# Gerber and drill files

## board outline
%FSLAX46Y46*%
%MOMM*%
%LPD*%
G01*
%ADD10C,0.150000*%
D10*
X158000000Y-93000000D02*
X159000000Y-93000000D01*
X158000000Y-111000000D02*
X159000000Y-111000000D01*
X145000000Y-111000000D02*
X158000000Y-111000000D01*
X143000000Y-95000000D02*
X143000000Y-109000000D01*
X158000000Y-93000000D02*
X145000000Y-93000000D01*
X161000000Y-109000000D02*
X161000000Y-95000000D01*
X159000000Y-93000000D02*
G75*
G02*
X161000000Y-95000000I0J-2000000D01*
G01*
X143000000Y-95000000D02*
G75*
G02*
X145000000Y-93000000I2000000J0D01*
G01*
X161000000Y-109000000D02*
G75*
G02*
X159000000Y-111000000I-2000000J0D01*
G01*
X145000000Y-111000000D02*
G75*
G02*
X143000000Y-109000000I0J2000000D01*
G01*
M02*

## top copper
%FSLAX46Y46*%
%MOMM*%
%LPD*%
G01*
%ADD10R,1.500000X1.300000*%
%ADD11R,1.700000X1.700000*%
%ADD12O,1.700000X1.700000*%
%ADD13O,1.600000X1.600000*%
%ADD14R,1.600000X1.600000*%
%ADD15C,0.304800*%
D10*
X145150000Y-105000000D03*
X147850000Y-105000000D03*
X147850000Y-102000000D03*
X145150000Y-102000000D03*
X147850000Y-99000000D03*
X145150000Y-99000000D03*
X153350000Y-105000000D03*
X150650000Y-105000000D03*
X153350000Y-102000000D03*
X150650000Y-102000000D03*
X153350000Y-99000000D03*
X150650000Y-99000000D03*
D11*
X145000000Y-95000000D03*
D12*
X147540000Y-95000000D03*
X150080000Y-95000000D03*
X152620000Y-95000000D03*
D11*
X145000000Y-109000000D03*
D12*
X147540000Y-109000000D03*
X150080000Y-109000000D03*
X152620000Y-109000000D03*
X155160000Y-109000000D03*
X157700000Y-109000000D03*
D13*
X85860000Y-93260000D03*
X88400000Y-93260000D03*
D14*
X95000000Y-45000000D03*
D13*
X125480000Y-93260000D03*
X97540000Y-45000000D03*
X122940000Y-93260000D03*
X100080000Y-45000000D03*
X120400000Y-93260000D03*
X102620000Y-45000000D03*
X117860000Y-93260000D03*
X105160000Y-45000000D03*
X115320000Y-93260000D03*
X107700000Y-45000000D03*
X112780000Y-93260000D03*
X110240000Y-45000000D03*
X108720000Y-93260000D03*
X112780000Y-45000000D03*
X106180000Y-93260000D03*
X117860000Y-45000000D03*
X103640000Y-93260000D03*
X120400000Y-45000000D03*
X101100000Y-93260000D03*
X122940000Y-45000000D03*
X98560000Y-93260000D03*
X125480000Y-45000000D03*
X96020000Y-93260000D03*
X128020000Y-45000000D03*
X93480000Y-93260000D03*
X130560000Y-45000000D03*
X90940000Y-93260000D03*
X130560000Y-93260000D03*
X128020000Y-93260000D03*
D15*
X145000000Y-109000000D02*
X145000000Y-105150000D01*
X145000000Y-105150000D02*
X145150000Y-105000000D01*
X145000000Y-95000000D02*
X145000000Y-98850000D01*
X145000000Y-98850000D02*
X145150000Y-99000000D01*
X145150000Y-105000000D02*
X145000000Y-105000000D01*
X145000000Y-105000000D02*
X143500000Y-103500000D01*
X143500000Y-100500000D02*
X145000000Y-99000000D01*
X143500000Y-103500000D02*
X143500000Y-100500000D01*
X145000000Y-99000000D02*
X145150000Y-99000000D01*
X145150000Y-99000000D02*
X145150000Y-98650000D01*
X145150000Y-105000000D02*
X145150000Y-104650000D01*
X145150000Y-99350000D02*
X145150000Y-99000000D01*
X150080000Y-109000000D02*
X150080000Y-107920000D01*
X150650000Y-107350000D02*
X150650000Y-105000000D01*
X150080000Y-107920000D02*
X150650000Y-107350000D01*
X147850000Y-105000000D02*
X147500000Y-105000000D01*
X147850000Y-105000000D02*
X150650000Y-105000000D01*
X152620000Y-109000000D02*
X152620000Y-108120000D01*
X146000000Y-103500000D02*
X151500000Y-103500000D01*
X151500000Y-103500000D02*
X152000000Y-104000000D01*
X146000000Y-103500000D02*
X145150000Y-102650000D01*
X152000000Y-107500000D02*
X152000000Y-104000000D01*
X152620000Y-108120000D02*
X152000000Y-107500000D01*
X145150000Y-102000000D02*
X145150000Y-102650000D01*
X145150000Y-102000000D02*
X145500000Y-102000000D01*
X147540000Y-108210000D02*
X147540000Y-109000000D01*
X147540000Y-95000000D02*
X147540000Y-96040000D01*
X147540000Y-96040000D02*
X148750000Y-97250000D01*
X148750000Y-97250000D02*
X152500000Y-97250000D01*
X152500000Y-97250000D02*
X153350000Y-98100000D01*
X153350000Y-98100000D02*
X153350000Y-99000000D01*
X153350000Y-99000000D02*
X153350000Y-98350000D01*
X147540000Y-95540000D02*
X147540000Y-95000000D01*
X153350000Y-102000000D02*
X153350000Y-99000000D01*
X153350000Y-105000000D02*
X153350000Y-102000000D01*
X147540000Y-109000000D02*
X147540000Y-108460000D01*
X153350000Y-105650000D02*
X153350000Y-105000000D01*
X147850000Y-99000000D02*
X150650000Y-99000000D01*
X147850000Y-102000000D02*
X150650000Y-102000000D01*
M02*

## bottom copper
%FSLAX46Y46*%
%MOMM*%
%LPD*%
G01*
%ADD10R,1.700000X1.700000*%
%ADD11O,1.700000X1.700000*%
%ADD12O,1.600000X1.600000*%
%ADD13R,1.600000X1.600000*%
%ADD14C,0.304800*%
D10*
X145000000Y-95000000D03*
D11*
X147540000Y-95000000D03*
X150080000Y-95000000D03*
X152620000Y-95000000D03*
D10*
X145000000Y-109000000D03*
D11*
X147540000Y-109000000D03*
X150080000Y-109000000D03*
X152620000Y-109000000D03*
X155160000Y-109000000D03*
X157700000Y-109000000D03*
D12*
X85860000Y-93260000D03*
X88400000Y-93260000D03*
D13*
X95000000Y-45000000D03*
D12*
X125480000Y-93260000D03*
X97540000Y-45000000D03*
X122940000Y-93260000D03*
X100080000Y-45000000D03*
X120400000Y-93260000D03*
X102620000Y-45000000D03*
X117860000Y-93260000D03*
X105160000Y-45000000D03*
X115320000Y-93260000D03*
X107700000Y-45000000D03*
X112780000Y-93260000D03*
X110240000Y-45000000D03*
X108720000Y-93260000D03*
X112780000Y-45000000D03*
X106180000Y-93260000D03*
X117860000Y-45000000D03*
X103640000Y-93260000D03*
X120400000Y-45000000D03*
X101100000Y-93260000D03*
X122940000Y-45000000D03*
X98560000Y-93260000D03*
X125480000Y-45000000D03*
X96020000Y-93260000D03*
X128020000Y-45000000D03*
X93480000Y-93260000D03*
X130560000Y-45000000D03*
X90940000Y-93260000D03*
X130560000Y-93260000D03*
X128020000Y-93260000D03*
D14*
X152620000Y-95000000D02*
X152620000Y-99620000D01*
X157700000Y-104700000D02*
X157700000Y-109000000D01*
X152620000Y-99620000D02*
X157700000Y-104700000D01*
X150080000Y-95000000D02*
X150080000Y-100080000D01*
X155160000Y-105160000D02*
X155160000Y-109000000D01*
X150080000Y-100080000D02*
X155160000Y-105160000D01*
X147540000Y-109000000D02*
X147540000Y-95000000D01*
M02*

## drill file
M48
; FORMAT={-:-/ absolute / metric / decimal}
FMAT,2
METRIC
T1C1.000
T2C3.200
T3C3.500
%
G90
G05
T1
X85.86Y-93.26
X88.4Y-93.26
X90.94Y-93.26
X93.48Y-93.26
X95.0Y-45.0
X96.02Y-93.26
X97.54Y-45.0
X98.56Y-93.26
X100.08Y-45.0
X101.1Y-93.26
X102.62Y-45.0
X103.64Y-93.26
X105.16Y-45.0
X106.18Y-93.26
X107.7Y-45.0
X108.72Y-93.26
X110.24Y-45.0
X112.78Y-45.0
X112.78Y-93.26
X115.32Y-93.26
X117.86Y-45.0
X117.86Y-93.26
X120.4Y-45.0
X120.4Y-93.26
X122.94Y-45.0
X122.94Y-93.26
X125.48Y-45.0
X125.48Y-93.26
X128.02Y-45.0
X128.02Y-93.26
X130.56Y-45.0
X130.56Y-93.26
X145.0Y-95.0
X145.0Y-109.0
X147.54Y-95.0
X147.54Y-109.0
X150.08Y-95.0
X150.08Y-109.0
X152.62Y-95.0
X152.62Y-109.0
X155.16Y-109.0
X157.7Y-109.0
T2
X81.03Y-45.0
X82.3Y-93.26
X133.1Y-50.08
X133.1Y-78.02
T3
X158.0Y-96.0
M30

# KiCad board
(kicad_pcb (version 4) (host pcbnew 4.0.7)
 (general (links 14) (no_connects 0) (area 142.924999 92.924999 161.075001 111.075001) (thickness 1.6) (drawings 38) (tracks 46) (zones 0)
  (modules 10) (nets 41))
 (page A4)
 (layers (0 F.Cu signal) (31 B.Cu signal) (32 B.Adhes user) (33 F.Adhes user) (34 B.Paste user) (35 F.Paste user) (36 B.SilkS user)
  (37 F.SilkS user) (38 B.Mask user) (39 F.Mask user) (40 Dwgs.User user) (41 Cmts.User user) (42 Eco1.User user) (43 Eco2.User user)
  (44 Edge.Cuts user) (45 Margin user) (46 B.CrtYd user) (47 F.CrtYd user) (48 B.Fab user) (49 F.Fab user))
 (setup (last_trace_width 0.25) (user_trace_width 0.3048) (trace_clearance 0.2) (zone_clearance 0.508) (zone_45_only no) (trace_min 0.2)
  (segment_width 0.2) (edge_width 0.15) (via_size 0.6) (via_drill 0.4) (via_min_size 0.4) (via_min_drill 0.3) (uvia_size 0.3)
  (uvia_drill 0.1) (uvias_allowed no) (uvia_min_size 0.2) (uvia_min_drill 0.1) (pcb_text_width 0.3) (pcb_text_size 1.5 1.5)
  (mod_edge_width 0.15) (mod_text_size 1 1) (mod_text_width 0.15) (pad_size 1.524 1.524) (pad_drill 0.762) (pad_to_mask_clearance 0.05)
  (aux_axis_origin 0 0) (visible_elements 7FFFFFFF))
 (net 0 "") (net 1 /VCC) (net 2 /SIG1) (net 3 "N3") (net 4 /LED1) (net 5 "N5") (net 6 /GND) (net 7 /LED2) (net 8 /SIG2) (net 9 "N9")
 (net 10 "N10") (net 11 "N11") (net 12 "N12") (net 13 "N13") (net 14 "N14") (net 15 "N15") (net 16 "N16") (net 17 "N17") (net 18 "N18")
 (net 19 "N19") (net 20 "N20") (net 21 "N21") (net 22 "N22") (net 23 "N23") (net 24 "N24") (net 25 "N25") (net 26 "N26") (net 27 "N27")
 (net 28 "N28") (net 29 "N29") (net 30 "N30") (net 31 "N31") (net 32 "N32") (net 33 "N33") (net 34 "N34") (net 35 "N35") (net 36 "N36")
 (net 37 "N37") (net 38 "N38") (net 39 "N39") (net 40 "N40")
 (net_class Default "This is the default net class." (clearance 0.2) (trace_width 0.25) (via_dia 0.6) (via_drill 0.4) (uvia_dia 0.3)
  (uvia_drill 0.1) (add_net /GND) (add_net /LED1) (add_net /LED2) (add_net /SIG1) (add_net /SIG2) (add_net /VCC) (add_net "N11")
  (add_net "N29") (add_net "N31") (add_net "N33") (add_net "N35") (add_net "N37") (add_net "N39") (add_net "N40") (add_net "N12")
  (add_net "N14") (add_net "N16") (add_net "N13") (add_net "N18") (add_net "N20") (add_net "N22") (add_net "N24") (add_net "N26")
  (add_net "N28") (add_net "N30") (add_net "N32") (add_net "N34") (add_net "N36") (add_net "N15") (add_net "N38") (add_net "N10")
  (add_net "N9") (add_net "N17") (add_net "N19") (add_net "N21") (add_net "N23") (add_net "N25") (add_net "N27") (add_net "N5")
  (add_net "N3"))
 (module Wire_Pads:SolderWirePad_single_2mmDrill (layer F.Cu) (at 158 96)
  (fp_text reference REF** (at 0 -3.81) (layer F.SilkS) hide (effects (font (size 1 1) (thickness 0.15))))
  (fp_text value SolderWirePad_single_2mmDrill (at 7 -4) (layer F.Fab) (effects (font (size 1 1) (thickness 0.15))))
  (pad "" np_thru_hole circle (at 0 0) (size 3.5 3.5) (drill 3.5) (layers *.Cu *.Mask)))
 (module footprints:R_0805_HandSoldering (layer F.Cu) (at 146.5 105)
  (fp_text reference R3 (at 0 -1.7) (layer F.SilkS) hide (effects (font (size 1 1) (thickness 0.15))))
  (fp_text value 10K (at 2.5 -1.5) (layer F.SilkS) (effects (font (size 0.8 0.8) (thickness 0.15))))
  (pad 1 smd rect (at -1.35 0) (size 1.5 1.3) (layers F.Cu F.Paste F.Mask) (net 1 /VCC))
  (pad 2 smd rect (at 1.35 0) (size 1.5 1.3) (layers F.Cu F.Paste F.Mask) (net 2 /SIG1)))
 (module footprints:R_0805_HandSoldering (layer F.Cu) (at 146.5 102 180)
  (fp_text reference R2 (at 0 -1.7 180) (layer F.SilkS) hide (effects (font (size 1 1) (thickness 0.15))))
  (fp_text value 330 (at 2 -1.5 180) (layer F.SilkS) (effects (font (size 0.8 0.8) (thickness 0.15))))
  (pad 1 smd rect (at -1.35 0 180) (size 1.5 1.3) (layers F.Cu F.Paste F.Mask) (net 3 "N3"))
  (pad 2 smd rect (at 1.35 0 180) (size 1.5 1.3) (layers F.Cu F.Paste F.Mask) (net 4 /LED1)))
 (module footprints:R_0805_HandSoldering (layer F.Cu) (at 146.5 99 180)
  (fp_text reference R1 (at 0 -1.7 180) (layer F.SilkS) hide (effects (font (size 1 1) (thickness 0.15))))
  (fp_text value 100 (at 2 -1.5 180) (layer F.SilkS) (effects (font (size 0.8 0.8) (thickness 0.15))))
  (pad 1 smd rect (at -1.35 0 180) (size 1.5 1.3) (layers F.Cu F.Paste F.Mask) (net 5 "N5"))
  (pad 2 smd rect (at 1.35 0 180) (size 1.5 1.3) (layers F.Cu F.Paste F.Mask) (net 1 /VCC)))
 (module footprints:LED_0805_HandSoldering (layer F.Cu) (at 152 105 180)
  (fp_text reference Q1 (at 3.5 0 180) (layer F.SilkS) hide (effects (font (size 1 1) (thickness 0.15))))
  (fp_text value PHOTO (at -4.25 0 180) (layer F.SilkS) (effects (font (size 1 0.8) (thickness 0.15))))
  (pad 1 smd rect (at -1.35 0 180) (size 1.5 1.3) (layers F.Cu F.Paste F.Mask) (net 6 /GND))
  (pad 2 smd rect (at 1.35 0 180) (size 1.5 1.3) (layers F.Cu F.Paste F.Mask) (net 2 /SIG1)))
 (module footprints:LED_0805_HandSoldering (layer F.Cu) (at 152 102 180)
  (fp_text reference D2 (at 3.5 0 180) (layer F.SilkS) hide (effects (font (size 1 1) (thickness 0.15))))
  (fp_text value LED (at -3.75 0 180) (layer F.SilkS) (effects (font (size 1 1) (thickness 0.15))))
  (pad 1 smd rect (at -1.35 0 180) (size 1.5 1.3) (layers F.Cu F.Paste F.Mask) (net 6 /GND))
  (pad 2 smd rect (at 1.35 0 180) (size 1.5 1.3) (layers F.Cu F.Paste F.Mask) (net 3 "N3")))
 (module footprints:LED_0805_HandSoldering (layer F.Cu) (at 152 99 180)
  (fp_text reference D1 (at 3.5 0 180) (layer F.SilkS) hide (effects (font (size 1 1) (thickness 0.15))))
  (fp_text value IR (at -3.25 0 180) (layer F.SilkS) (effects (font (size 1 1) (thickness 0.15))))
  (pad 1 smd rect (at -1.35 0 180) (size 1.5 1.3) (layers F.Cu F.Paste F.Mask) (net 6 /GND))
  (pad 2 smd rect (at 1.35 0 180) (size 1.5 1.3) (layers F.Cu F.Paste F.Mask) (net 5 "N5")))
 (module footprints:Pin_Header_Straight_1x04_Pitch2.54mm (layer F.Cu) (at 145 95 90)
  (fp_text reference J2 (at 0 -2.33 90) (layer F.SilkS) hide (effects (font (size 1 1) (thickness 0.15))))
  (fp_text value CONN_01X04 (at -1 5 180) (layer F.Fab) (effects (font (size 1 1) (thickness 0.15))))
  (pad 1 thru_hole rect (at 0 0 90) (size 1.7 1.7) (drill 1) (layers *.Cu *.Mask) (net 1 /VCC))
  (pad 2 thru_hole oval (at 0 2.54 90) (size 1.7 1.7) (drill 1) (layers *.Cu *.Mask) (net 6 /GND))
  (pad 3 thru_hole oval (at 0 5.08 90) (size 1.7 1.7) (drill 1) (layers *.Cu *.Mask) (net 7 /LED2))
  (pad 4 thru_hole oval (at 0 7.62 90) (size 1.7 1.7) (drill 1) (layers *.Cu *.Mask) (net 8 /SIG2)))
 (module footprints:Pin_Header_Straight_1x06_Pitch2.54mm (layer F.Cu) (at 145 109 90)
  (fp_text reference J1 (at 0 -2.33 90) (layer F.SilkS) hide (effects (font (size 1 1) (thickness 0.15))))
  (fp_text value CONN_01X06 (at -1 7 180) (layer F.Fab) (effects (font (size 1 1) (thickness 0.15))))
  (pad 1 thru_hole rect (at 0 0 90) (size 1.7 1.7) (drill 1) (layers *.Cu *.Mask) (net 1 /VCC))
  (pad 2 thru_hole oval (at 0 2.54 90) (size 1.7 1.7) (drill 1) (layers *.Cu *.Mask) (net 6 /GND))
  (pad 3 thru_hole oval (at 0 5.08 90) (size 1.7 1.7) (drill 1) (layers *.Cu *.Mask) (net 2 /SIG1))
  (pad 4 thru_hole oval (at 0 7.62 90) (size 1.7 1.7) (drill 1) (layers *.Cu *.Mask) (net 4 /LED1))
  (pad 5 thru_hole oval (at 0 10.16 90) (size 1.7 1.7) (drill 1) (layers *.Cu *.Mask) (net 7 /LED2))
  (pad 6 thru_hole oval (at 0 12.7 90) (size 1.7 1.7) (drill 1) (layers *.Cu *.Mask) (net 8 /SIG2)))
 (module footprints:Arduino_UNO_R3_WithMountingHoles (layer F.Cu) (at 95 45)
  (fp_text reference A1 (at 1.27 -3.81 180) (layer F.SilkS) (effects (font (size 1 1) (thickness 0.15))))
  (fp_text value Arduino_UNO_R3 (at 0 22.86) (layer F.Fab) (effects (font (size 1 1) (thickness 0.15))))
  (pad 32 thru_hole oval (at -9.14 48.26 90) (size 1.6 1.6) (drill 1) (layers *.Cu *.Mask) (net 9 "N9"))
  (pad 31 thru_hole oval (at -6.6 48.26 90) (size 1.6 1.6) (drill 1) (layers *.Cu *.Mask) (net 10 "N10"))
  (pad 1 thru_hole rect (at 0 0 90) (size 1.6 1.6) (drill 1) (layers *.Cu *.Mask) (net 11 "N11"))
  (pad 17 thru_hole oval (at 30.48 48.26 90) (size 1.6 1.6) (drill 1) (layers *.Cu *.Mask) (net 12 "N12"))
  (pad 2 thru_hole oval (at 2.54 0 90) (size 1.6 1.6) (drill 1) (layers *.Cu *.Mask) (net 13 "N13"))
  (pad 18 thru_hole oval (at 27.94 48.26 90) (size 1.6 1.6) (drill 1) (layers *.Cu *.Mask) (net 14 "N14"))
  (pad 3 thru_hole oval (at 5.08 0 90) (size 1.6 1.6) (drill 1) (layers *.Cu *.Mask) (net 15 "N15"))
  (pad 19 thru_hole oval (at 25.4 48.26 90) (size 1.6 1.6) (drill 1) (layers *.Cu *.Mask) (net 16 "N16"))
  (pad 4 thru_hole oval (at 7.62 0 90) (size 1.6 1.6) (drill 1) (layers *.Cu *.Mask) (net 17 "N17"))
  (pad 20 thru_hole oval (at 22.86 48.26 90) (size 1.6 1.6) (drill 1) (layers *.Cu *.Mask) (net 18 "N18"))
  (pad 5 thru_hole oval (at 10.16 0 90) (size 1.6 1.6) (drill 1) (layers *.Cu *.Mask) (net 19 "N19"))
  (pad 21 thru_hole oval (at 20.32 48.26 90) (size 1.6 1.6) (drill 1) (layers *.Cu *.Mask) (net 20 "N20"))
  (pad 6 thru_hole oval (at 12.7 0 90) (size 1.6 1.6) (drill 1) (layers *.Cu *.Mask) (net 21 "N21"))
  (pad 22 thru_hole oval (at 17.78 48.26 90) (size 1.6 1.6) (drill 1) (layers *.Cu *.Mask) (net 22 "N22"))
  (pad 7 thru_hole oval (at 15.24 0 90) (size 1.6 1.6) (drill 1) (layers *.Cu *.Mask) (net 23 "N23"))
  (pad 23 thru_hole oval (at 13.72 48.26 90) (size 1.6 1.6) (drill 1) (layers *.Cu *.Mask) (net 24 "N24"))
  (pad 8 thru_hole oval (at 17.78 0 90) (size 1.6 1.6) (drill 1) (layers *.Cu *.Mask) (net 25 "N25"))
  (pad 24 thru_hole oval (at 11.18 48.26 90) (size 1.6 1.6) (drill 1) (layers *.Cu *.Mask) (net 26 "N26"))
  (pad 9 thru_hole oval (at 22.86 0 90) (size 1.6 1.6) (drill 1) (layers *.Cu *.Mask) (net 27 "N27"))
  (pad 25 thru_hole oval (at 8.64 48.26 90) (size 1.6 1.6) (drill 1) (layers *.Cu *.Mask) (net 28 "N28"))
  (pad 10 thru_hole oval (at 25.4 0 90) (size 1.6 1.6) (drill 1) (layers *.Cu *.Mask) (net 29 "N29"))
  (pad 26 thru_hole oval (at 6.1 48.26 90) (size 1.6 1.6) (drill 1) (layers *.Cu *.Mask) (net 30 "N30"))
  (pad 11 thru_hole oval (at 27.94 0 90) (size 1.6 1.6) (drill 1) (layers *.Cu *.Mask) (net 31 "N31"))
  (pad 27 thru_hole oval (at 3.56 48.26 90) (size 1.6 1.6) (drill 1) (layers *.Cu *.Mask) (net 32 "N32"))
  (pad 12 thru_hole oval (at 30.48 0 90) (size 1.6 1.6) (drill 1) (layers *.Cu *.Mask) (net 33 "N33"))
  (pad 28 thru_hole oval (at 1.02 48.26 90) (size 1.6 1.6) (drill 1) (layers *.Cu *.Mask) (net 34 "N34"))
  (pad 13 thru_hole oval (at 33.02 0 90) (size 1.6 1.6) (drill 1) (layers *.Cu *.Mask) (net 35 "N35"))
  (pad 29 thru_hole oval (at -1.52 48.26 90) (size 1.6 1.6) (drill 1) (layers *.Cu *.Mask) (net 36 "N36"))
  (pad 14 thru_hole oval (at 35.56 0 90) (size 1.6 1.6) (drill 1) (layers *.Cu *.Mask) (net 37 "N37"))
  (pad 30 thru_hole oval (at -4.06 48.26 90) (size 1.6 1.6) (drill 1) (layers *.Cu *.Mask) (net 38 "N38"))
  (pad 15 thru_hole oval (at 35.56 48.26 90) (size 1.6 1.6) (drill 1) (layers *.Cu *.Mask) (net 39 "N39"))
  (pad 16 thru_hole oval (at 33.02 48.26 90) (size 1.6 1.6) (drill 1) (layers *.Cu *.Mask) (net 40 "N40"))
  (pad "" np_thru_hole circle (at -13.97 0 90) (size 3.2 3.2) (drill 3.2) (layers *.Cu *.Mask))
  (pad "" np_thru_hole circle (at -12.7 48.26 90) (size 3.2 3.2) (drill 3.2) (layers *.Cu *.Mask))
  (pad "" np_thru_hole circle (at 38.1 33.02 90) (size 3.2 3.2) (drill 3.2) (layers *.Cu *.Mask))
  (pad "" np_thru_hole circle (at 38.1 5.08 90) (size 3.2 3.2) (drill 3.2) (layers *.Cu *.Mask)))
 (gr_line (start 158 93) (end 159 93) (angle 90) (layer Edge.Cuts) (width 0.15))
 (gr_line (start 158 111) (end 159 111) (angle 90) (layer Edge.Cuts) (width 0.15))
 (gr_line (start 145 111) (end 158 111) (angle 90) (layer Edge.Cuts) (width 0.15))
 (gr_line (start 143 95) (end 143 109) (angle 90) (layer Edge.Cuts) (width 0.15))
 (gr_line (start 158 93) (end 145 93) (angle 90) (layer Edge.Cuts) (width 0.15))
 (gr_line (start 161 109) (end 161 95) (angle 90) (layer Edge.Cuts) (width 0.15))
 (gr_arc (start 159 95) (end 159 93) (angle 90) (layer Edge.Cuts) (width 0.15))
 (gr_arc (start 145 95) (end 143 95) (angle 90) (layer Edge.Cuts) (width 0.15))
 (gr_arc (start 159 109) (end 161 109) (angle 90) (layer Edge.Cuts) (width 0.15))
 (gr_arc (start 145 109) (end 145 111) (angle 90) (layer Edge.Cuts) (width 0.15))
 (segment (start 145 109) (end 145 105.15) (width 0.3048) (layer F.Cu) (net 1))
 (segment (start 145 105.15) (end 145.15 105) (width 0.3048) (layer F.Cu) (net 1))
 (segment (start 145 95) (end 145 98.85) (width 0.3048) (layer F.Cu) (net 1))
 (segment (start 145 98.85) (end 145.15 99) (width 0.3048) (layer F.Cu) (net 1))
 (segment (start 145.15 105) (end 145 105) (width 0.3048) (layer F.Cu) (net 1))
 (segment (start 145 105) (end 143.5 103.5) (width 0.3048) (layer F.Cu) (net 1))
 (segment (start 143.5 100.5) (end 145 99) (width 0.3048) (layer F.Cu) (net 1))
 (segment (start 143.5 103.5) (end 143.5 100.5) (width 0.3048) (layer F.Cu) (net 1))
 (segment (start 145 99) (end 145.15 99) (width 0.3048) (layer F.Cu) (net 1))
 (segment (start 145.15 99) (end 145.15 98.65) (width 0.3048) (layer F.Cu) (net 1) (status 30))
 (segment (start 145.15 105) (end 145.15 104.65) (width 0.3048) (layer F.Cu) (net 1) (status 30))
 (segment (start 145.15 99.35) (end 145.15 99) (width 0.3048) (layer F.Cu) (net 1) (status 30))
 (segment (start 150.08 109) (end 150.08 107.92) (width 0.3048) (layer F.Cu) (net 2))
 (segment (start 150.65 107.35) (end 150.65 105) (width 0.3048) (layer F.Cu) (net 2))
 (segment (start 150.08 107.92) (end 150.65 107.35) (width 0.3048) (layer F.Cu) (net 2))
 (segment (start 147.85 105) (end 147.5 105) (width 0.3048) (layer F.Cu) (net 2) (status 30))
 (segment (start 147.85 105) (end 150.65 105) (width 0.3048) (layer F.Cu) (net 2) (status 10))
 (segment (start 152.62 95) (end 152.62 99.62) (width 0.3048) (layer B.Cu) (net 8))
 (segment (start 157.7 104.7) (end 157.7 109) (width 0.3048) (layer B.Cu) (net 8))
 (segment (start 152.62 99.62) (end 157.7 104.7) (width 0.3048) (layer B.Cu) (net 8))
 (segment (start 152.62 109) (end 152.62 108.12) (width 0.3048) (layer F.Cu) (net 4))
 (segment (start 146 103.5) (end 151.5 103.5) (width 0.3048) (layer F.Cu) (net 4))
 (segment (start 151.5 103.5) (end 152 104) (width 0.3048) (layer F.Cu) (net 4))
 (segment (start 146 103.5) (end 145.15 102.65) (width 0.3048) (layer F.Cu) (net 4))
 (segment (start 152 107.5) (end 152 104) (width 0.3048) (layer F.Cu) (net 4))
 (segment (start 152.62 108.12) (end 152 107.5) (width 0.3048) (layer F.Cu) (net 4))
 (segment (start 145.15 102) (end 145.15 102.65) (width 0.3048) (layer F.Cu) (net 4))
 (segment (start 145.15 102) (end 145.5 102) (width 0.3048) (layer F.Cu) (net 4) (status 30))
 (segment (start 150.08 95) (end 150.08 100.08) (width 0.3048) (layer B.Cu) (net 7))
 (segment (start 155.16 105.16) (end 155.16 109) (width 0.3048) (layer B.Cu) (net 7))
 (segment (start 150.08 100.08) (end 155.16 105.16) (width 0.3048) (layer B.Cu) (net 7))
 (segment (start 147.54 109) (end 147.54 95) (width 0.3048) (layer B.Cu) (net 6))
 (segment (start 147.54 108.21) (end 147.54 109) (width 0.3048) (layer F.Cu) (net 6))
 (segment (start 147.54 95) (end 147.54 96.04) (width 0.3048) (layer F.Cu) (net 6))
 (segment (start 147.54 96.04) (end 148.75 97.25) (width 0.3048) (layer F.Cu) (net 6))
 (segment (start 148.75 97.25) (end 152.5 97.25) (width 0.3048) (layer F.Cu) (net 6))
 (segment (start 152.5 97.25) (end 153.35 98.1) (width 0.3048) (layer F.Cu) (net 6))
 (segment (start 153.35 98.1) (end 153.35 99) (width 0.3048) (layer F.Cu) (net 6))
 (segment (start 153.35 99) (end 153.35 98.35) (width 0.3048) (layer F.Cu) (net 6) (status 30))
 (segment (start 147.54 95.54) (end 147.54 95) (width 0.3048) (layer F.Cu) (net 6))
 (segment (start 153.35 102) (end 153.35 99) (width 0.3048) (layer F.Cu) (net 6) (status 20))
 (segment (start 153.35 105) (end 153.35 102) (width 0.3048) (layer F.Cu) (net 6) (status 10))
 (segment (start 147.54 109) (end 147.54 108.46) (width 0.3048) (layer F.Cu) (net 6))
 (segment (start 153.35 105.65) (end 153.35 105) (width 0.3048) (layer F.Cu) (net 6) (status 30))
 (segment (start 147.85 99) (end 150.65 99) (width 0.3048) (layer F.Cu) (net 5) (status 10))
 (segment (start 147.85 102) (end 150.65 102) (width 0.3048) (layer F.Cu) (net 3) (status 10)))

